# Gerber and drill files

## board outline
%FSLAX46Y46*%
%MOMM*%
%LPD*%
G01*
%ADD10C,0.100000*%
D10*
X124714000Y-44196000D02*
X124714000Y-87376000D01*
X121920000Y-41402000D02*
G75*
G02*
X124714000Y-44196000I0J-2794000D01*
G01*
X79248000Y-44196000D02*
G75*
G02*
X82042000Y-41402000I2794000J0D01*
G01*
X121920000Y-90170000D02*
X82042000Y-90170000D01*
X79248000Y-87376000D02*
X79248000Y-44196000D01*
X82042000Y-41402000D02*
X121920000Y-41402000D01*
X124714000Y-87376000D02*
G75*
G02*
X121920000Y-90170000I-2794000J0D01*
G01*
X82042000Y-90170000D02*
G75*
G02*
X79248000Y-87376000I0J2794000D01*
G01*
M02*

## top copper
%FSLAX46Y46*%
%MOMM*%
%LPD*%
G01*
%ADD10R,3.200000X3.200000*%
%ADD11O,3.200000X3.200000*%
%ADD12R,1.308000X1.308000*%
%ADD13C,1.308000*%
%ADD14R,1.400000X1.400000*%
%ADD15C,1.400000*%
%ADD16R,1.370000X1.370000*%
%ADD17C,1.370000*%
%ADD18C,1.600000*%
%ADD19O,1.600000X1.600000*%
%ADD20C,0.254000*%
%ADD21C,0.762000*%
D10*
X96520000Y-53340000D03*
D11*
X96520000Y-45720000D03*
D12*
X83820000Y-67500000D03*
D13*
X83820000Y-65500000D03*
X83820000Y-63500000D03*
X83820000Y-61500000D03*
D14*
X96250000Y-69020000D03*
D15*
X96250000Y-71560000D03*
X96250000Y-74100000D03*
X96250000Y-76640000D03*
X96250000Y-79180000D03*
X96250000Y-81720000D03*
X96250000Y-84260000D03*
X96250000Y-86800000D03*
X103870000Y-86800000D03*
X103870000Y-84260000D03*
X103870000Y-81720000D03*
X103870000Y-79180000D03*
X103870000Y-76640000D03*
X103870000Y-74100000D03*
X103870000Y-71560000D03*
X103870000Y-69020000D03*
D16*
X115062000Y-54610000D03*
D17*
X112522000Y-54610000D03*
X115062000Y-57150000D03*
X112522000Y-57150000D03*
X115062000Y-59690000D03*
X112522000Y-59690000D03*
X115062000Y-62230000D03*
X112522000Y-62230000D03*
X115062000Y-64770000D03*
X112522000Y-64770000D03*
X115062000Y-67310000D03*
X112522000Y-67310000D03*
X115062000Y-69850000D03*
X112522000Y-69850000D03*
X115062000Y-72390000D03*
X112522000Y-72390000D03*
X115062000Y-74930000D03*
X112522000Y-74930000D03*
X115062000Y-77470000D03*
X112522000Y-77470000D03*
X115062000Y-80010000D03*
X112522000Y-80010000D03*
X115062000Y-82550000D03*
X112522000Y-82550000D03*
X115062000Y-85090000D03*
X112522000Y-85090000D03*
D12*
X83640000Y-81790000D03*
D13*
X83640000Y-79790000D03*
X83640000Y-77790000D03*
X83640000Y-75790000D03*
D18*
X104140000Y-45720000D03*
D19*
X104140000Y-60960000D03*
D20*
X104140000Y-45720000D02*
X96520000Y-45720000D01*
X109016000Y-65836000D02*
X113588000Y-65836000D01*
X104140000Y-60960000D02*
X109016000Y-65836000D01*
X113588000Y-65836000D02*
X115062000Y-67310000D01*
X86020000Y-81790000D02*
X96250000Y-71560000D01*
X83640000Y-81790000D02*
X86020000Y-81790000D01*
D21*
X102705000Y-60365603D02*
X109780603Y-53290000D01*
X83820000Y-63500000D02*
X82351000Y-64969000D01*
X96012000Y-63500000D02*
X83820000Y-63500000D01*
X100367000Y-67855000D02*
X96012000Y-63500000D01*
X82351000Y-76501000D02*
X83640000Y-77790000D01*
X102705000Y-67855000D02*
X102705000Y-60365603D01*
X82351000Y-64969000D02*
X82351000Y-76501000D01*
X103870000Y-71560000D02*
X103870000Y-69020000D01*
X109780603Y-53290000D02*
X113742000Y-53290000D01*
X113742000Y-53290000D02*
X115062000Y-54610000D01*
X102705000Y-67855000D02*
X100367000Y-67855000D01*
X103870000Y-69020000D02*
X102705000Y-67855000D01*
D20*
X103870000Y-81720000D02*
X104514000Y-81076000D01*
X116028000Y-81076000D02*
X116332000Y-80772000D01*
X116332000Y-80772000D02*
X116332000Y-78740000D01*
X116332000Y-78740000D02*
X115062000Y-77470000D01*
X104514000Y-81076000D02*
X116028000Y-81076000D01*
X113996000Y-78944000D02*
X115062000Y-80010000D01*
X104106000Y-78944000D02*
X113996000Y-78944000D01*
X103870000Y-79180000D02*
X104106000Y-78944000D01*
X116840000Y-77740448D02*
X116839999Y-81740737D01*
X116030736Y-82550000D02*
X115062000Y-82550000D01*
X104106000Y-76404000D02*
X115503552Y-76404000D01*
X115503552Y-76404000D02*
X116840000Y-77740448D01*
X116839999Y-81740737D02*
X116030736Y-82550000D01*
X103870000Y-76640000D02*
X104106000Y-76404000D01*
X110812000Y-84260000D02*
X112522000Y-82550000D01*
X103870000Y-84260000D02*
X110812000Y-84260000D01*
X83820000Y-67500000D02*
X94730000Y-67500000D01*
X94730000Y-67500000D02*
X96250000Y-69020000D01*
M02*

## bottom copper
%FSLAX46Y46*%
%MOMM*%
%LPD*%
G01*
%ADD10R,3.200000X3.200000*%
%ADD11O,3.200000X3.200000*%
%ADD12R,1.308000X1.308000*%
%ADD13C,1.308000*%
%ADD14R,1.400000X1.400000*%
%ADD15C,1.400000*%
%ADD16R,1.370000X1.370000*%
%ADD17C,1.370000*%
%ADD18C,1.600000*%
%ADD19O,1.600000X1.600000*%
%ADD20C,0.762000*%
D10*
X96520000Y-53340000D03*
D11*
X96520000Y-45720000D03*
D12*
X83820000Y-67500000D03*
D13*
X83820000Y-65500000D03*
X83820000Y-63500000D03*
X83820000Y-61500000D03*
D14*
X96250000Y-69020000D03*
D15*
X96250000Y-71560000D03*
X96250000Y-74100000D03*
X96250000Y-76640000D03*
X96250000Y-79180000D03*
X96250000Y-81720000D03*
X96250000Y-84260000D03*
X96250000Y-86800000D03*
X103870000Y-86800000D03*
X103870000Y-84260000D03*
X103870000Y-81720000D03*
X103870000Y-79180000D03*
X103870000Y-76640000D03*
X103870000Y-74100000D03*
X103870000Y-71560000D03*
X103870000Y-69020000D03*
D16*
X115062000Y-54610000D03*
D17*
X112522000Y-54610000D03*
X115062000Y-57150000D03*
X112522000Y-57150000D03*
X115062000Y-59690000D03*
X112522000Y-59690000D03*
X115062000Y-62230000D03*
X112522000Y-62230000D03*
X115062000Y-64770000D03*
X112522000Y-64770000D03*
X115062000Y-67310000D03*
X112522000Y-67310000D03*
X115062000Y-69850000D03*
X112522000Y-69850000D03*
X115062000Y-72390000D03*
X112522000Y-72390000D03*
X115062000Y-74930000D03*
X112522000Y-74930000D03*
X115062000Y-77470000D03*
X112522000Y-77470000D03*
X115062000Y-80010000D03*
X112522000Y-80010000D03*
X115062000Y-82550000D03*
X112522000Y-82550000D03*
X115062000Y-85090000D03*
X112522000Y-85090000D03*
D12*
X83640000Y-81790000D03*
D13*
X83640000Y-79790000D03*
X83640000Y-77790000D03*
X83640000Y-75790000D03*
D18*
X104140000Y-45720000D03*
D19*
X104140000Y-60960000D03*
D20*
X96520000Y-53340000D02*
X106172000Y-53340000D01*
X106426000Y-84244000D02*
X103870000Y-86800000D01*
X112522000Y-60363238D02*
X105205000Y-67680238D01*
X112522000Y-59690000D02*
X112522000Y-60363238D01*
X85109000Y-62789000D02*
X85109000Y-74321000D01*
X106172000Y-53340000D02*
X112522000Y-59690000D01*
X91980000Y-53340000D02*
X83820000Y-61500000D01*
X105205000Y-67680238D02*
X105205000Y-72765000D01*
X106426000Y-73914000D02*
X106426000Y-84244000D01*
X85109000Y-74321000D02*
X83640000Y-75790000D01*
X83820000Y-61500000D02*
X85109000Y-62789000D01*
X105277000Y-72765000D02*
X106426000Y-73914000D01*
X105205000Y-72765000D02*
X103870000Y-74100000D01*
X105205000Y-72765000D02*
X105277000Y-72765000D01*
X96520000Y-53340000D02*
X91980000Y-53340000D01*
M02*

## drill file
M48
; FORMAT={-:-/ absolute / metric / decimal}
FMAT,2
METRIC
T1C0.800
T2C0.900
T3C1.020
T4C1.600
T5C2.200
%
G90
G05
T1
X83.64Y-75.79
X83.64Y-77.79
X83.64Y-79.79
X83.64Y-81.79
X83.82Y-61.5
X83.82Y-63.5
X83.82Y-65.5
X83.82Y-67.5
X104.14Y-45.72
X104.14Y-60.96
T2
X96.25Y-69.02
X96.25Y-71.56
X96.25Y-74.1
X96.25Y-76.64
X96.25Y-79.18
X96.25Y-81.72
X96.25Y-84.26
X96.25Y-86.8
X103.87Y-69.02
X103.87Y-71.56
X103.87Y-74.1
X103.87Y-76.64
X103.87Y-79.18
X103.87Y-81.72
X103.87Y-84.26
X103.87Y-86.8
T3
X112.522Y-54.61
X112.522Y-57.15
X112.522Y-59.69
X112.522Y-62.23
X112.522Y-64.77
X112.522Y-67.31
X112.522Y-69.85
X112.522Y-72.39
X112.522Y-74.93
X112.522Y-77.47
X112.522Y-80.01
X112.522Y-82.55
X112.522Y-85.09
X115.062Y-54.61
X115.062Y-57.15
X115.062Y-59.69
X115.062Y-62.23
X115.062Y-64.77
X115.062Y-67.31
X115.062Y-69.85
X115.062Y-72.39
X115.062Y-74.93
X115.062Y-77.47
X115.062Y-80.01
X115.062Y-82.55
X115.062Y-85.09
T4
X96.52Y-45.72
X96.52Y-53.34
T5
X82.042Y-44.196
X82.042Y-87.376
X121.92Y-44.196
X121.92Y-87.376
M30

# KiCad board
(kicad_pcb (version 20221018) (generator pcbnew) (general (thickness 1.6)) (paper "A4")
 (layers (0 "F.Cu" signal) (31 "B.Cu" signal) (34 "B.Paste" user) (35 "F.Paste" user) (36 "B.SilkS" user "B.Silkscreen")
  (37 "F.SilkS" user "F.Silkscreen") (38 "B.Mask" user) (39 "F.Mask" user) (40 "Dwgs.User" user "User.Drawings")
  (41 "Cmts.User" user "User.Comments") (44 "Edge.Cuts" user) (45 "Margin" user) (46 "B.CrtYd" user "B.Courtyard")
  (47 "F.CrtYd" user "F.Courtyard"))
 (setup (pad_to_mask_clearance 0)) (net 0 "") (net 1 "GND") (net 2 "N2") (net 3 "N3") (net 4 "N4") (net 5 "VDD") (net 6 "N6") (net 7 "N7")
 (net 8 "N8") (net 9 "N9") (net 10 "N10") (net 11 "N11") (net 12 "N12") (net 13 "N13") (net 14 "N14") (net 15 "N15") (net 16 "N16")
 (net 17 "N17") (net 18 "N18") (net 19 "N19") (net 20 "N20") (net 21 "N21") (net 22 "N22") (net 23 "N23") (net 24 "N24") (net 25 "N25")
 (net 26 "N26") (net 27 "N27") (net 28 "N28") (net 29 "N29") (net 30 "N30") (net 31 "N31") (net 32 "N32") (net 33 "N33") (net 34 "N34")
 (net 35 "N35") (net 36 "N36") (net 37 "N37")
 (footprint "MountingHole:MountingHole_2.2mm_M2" (layer "F.Cu") (at 121.92 44.196)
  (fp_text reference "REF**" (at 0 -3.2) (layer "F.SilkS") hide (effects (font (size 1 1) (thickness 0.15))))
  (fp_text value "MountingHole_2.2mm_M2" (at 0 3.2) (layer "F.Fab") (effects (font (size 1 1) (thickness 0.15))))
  (pad "" np_thru_hole circle (at 0 0) (size 2.2 2.2) (drill 2.2) (layers "*.Cu" "*.Mask")))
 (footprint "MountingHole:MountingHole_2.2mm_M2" (layer "F.Cu") (at 82.042 87.376)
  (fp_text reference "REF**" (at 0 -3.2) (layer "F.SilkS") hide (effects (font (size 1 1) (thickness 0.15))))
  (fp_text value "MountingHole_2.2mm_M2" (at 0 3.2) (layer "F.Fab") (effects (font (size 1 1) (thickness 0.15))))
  (pad "" np_thru_hole circle (at 0 0) (size 2.2 2.2) (drill 2.2) (layers "*.Cu" "*.Mask")))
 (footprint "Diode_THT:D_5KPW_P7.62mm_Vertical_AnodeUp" (layer "F.Cu") (at 96.52 53.34 90)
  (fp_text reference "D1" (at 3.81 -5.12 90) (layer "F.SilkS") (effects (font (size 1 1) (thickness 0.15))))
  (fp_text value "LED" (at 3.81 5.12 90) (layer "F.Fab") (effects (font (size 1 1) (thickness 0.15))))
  (pad "1" thru_hole rect (at 0 0 90) (size 3.2 3.2) (drill 1.6) (layers "*.Cu" "*.Mask") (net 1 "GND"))
  (pad "2" thru_hole oval (at 7.62 0 90) (size 3.2 3.2) (drill 1.6) (layers "*.Cu" "*.Mask") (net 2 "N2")))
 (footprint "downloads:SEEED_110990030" (layer "F.Cu") (at 83.82 64.5 90)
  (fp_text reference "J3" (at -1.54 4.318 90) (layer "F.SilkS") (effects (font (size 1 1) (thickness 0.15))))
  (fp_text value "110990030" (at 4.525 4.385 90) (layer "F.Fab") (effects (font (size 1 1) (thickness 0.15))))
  (pad "1" thru_hole rect (at -3 0 90) (size 1.308 1.308) (drill 0.8) (layers "*.Cu" "*.Mask") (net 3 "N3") (solder_mask_margin 0.102))
  (pad "2" thru_hole circle (at -1 0 90) (size 1.308 1.308) (drill 0.8) (layers "*.Cu" "*.Mask") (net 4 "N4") (solder_mask_margin 0.102))
  (pad "3" thru_hole circle (at 1 0 90) (size 1.308 1.308) (drill 0.8) (layers "*.Cu" "*.Mask") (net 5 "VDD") (solder_mask_margin 0.102))
  (pad "4" thru_hole circle (at 3 0 90) (size 1.308 1.308) (drill 0.8) (layers "*.Cu" "*.Mask") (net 1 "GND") (solder_mask_margin 0.102)))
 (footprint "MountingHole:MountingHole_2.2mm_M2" (layer "F.Cu") (at 82.042 44.196)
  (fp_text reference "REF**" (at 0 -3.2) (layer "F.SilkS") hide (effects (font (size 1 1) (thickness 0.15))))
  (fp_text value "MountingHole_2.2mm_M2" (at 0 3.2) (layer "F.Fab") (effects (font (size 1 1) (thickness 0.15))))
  (pad "" np_thru_hole circle (at 0 0) (size 2.2 2.2) (drill 2.2) (layers "*.Cu" "*.Mask")))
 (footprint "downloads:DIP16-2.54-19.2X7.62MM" (layer "F.Cu") (at 100.06 77.91 -90)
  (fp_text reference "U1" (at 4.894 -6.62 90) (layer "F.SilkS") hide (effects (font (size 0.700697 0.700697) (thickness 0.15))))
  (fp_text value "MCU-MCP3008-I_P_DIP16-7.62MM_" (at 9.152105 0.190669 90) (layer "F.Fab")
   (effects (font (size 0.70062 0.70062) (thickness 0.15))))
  (pad "1" thru_hole rect (at -8.89 3.81 270) (size 1.4 1.4) (drill 0.9) (layers "*.Cu" "*.Mask") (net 3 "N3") (solder_mask_margin 0.102))
  (pad "2" thru_hole circle (at -6.35 3.81 270) (size 1.4 1.4) (drill 0.9) (layers "*.Cu" "*.Mask") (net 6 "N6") (solder_mask_margin 0.102))
  (pad "3" thru_hole circle (at -3.81 3.81 270) (size 1.4 1.4) (drill 0.9) (layers "*.Cu" "*.Mask") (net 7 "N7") (solder_mask_margin 0.102))
  (pad "4" thru_hole circle (at -1.27 3.81 270) (size 1.4 1.4) (drill 0.9) (layers "*.Cu" "*.Mask") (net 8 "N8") (solder_mask_margin 0.102))
  (pad "5" thru_hole circle (at 1.27 3.81 270) (size 1.4 1.4) (drill 0.9) (layers "*.Cu" "*.Mask") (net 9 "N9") (solder_mask_margin 0.102))
  (pad "6" thru_hole circle (at 3.81 3.81 270) (size 1.4 1.4) (drill 0.9) (layers "*.Cu" "*.Mask") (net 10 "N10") (solder_mask_margin 0.102))
  (pad "7" thru_hole circle (at 6.35 3.81 270) (size 1.4 1.4) (drill 0.9) (layers "*.Cu" "*.Mask") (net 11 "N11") (solder_mask_margin 0.102))
  (pad "8" thru_hole circle (at 8.89 3.81 270) (size 1.4 1.4) (drill 0.9) (layers "*.Cu" "*.Mask") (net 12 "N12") (solder_mask_margin 0.102))
  (pad "9" thru_hole circle (at 8.89 -3.81 270) (size 1.4 1.4) (drill 0.9) (layers "*.Cu" "*.Mask") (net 1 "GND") (solder_mask_margin 0.102))
  (pad "10" thru_hole circle (at 6.35 -3.81 270) (size 1.4 1.4) (drill 0.9) (layers "*.Cu" "*.Mask") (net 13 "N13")
   (solder_mask_margin 0.102))
  (pad "11" thru_hole circle (at 3.81 -3.81 270) (size 1.4 1.4) (drill 0.9) (layers "*.Cu" "*.Mask") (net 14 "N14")
   (solder_mask_margin 0.102))
  (pad "12" thru_hole circle (at 1.27 -3.81 270) (size 1.4 1.4) (drill 0.9) (layers "*.Cu" "*.Mask") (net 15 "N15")
   (solder_mask_margin 0.102))
  (pad "13" thru_hole circle (at -1.27 -3.81 270) (size 1.4 1.4) (drill 0.9) (layers "*.Cu" "*.Mask") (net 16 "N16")
   (solder_mask_margin 0.102))
  (pad "14" thru_hole circle (at -3.81 -3.81 270) (size 1.4 1.4) (drill 0.9) (layers "*.Cu" "*.Mask") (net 1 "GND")
   (solder_mask_margin 0.102))
  (pad "15" thru_hole circle (at -6.35 -3.81 270) (size 1.4 1.4) (drill 0.9) (layers "*.Cu" "*.Mask") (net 5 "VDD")
   (solder_mask_margin 0.102))
  (pad "16" thru_hole circle (at -8.89 -3.81 270) (size 1.4 1.4) (drill 0.9) (layers "*.Cu" "*.Mask") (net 5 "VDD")
   (solder_mask_margin 0.102)))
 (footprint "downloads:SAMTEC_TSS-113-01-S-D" (layer "F.Cu") (at 112.912 54.61 -90)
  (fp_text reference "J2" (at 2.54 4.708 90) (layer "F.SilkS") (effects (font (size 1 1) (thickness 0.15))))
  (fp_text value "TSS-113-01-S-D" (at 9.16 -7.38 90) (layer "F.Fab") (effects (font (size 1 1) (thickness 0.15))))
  (pad "01" thru_hole rect (at 0 -2.15 270) (size 1.37 1.37) (drill 1.02) (layers "*.Cu" "*.Mask") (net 5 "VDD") (solder_mask_margin 0.102))
  (pad "02" thru_hole circle (at 0 0.39 270) (size 1.37 1.37) (drill 1.02) (layers "*.Cu" "*.Mask") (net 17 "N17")
   (solder_mask_margin 0.102))
  (pad "03" thru_hole circle (at 2.54 -2.15 270) (size 1.37 1.37) (drill 1.02) (layers "*.Cu" "*.Mask") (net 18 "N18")
   (solder_mask_margin 0.102))
  (pad "04" thru_hole circle (at 2.54 0.39 270) (size 1.37 1.37) (drill 1.02) (layers "*.Cu" "*.Mask") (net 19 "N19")
   (solder_mask_margin 0.102))
  (pad "05" thru_hole circle (at 5.08 -2.15 270) (size 1.37 1.37) (drill 1.02) (layers "*.Cu" "*.Mask") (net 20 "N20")
   (solder_mask_margin 0.102))
  (pad "06" thru_hole circle (at 5.08 0.39 270) (size 1.37 1.37) (drill 1.02) (layers "*.Cu" "*.Mask") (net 1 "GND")
   (solder_mask_margin 0.102))
  (pad "07" thru_hole circle (at 7.62 -2.15 270) (size 1.37 1.37) (drill 1.02) (layers "*.Cu" "*.Mask") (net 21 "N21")
   (solder_mask_margin 0.102))
  (pad "08" thru_hole circle (at 7.62 0.39 270) (size 1.37 1.37) (drill 1.02) (layers "*.Cu" "*.Mask") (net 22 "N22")
   (solder_mask_margin 0.102))
  (pad "09" thru_hole circle (at 10.16 -2.15 270) (size 1.37 1.37) (drill 1.02) (layers "*.Cu" "*.Mask") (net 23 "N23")
   (solder_mask_margin 0.102))
  (pad "10" thru_hole circle (at 10.16 0.39 270) (size 1.37 1.37) (drill 1.02) (layers "*.Cu" "*.Mask") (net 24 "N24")
   (solder_mask_margin 0.102))
  (pad "11" thru_hole circle (at 12.7 -2.15 270) (size 1.37 1.37) (drill 1.02) (layers "*.Cu" "*.Mask") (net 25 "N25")
   (solder_mask_margin 0.102))
  (pad "12" thru_hole circle (at 12.7 0.39 270) (size 1.37 1.37) (drill 1.02) (layers "*.Cu" "*.Mask") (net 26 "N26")
   (solder_mask_margin 0.102))
  (pad "13" thru_hole circle (at 15.24 -2.15 270) (size 1.37 1.37) (drill 1.02) (layers "*.Cu" "*.Mask") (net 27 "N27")
   (solder_mask_margin 0.102))
  (pad "14" thru_hole circle (at 15.24 0.39 270) (size 1.37 1.37) (drill 1.02) (layers "*.Cu" "*.Mask") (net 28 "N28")
   (solder_mask_margin 0.102))
  (pad "15" thru_hole circle (at 17.78 -2.15 270) (size 1.37 1.37) (drill 1.02) (layers "*.Cu" "*.Mask") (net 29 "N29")
   (solder_mask_margin 0.102))
  (pad "16" thru_hole circle (at 17.78 0.39 270) (size 1.37 1.37) (drill 1.02) (layers "*.Cu" "*.Mask") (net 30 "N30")
   (solder_mask_margin 0.102))
  (pad "17" thru_hole circle (at 20.32 -2.15 270) (size 1.37 1.37) (drill 1.02) (layers "*.Cu" "*.Mask") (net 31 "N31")
   (solder_mask_margin 0.102))
  (pad "18" thru_hole circle (at 20.32 0.39 270) (size 1.37 1.37) (drill 1.02) (layers "*.Cu" "*.Mask") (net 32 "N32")
   (solder_mask_margin 0.102))
  (pad "19" thru_hole circle (at 22.86 -2.15 270) (size 1.37 1.37) (drill 1.02) (layers "*.Cu" "*.Mask") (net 14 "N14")
   (solder_mask_margin 0.102))
  (pad "20" thru_hole circle (at 22.86 0.39 270) (size 1.37 1.37) (drill 1.02) (layers "*.Cu" "*.Mask") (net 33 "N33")
   (solder_mask_margin 0.102))
  (pad "21" thru_hole circle (at 25.4 -2.15 270) (size 1.37 1.37) (drill 1.02) (layers "*.Cu" "*.Mask") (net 15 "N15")
   (solder_mask_margin 0.102))
  (pad "22" thru_hole circle (at 25.4 0.39 270) (size 1.37 1.37) (drill 1.02) (layers "*.Cu" "*.Mask") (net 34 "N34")
   (solder_mask_margin 0.102))
  (pad "23" thru_hole circle (at 27.94 -2.15 270) (size 1.37 1.37) (drill 1.02) (layers "*.Cu" "*.Mask") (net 16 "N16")
   (solder_mask_margin 0.102))
  (pad "24" thru_hole circle (at 27.94 0.39 270) (size 1.37 1.37) (drill 1.02) (layers "*.Cu" "*.Mask") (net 13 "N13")
   (solder_mask_margin 0.102))
  (pad "25" thru_hole circle (at 30.48 -2.15 270) (size 1.37 1.37) (drill 1.02) (layers "*.Cu" "*.Mask") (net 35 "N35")
   (solder_mask_margin 0.102))
  (pad "26" thru_hole circle (at 30.48 0.39 270) (size 1.37 1.37) (drill 1.02) (layers "*.Cu" "*.Mask") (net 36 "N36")
   (solder_mask_margin 0.102)))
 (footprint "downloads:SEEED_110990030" (layer "F.Cu") (at 83.64 78.79 90)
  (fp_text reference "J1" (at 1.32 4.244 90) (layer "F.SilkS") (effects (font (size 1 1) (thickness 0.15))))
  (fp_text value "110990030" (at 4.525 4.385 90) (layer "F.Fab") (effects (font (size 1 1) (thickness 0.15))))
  (pad "1" thru_hole rect (at -3 0 90) (size 1.308 1.308) (drill 0.8) (layers "*.Cu" "*.Mask") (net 6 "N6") (solder_mask_margin 0.102))
  (pad "2" thru_hole circle (at -1 0 90) (size 1.308 1.308) (drill 0.8) (layers "*.Cu" "*.Mask") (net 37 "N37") (solder_mask_margin 0.102))
  (pad "3" thru_hole circle (at 1 0 90) (size 1.308 1.308) (drill 0.8) (layers "*.Cu" "*.Mask") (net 5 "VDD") (solder_mask_margin 0.102))
  (pad "4" thru_hole circle (at 3 0 90) (size 1.308 1.308) (drill 0.8) (layers "*.Cu" "*.Mask") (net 1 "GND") (solder_mask_margin 0.102)))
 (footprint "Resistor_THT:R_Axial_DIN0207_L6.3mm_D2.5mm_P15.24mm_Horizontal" (layer "F.Cu") (at 104.14 45.72 -90)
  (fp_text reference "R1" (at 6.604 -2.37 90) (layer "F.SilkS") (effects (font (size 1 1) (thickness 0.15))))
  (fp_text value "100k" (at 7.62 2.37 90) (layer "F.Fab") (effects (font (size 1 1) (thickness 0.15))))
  (pad "1" thru_hole circle (at 0 0 270) (size 1.6 1.6) (drill 0.8) (layers "*.Cu" "*.Mask") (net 2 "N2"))
  (pad "2" thru_hole oval (at 15.24 0 270) (size 1.6 1.6) (drill 0.8) (layers "*.Cu" "*.Mask") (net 25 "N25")))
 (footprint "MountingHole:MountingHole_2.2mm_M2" (layer "F.Cu") (at 121.92 87.376)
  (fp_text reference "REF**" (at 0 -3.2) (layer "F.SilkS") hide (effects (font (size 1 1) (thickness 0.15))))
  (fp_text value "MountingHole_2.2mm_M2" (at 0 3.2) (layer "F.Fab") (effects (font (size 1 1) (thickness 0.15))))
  (pad "" np_thru_hole circle (at 0 0) (size 2.2 2.2) (drill 2.2) (layers "*.Cu" "*.Mask")))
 (gr_line (start 124.714 44.196) (end 124.714 87.376) (stroke (width 0.1) (type default)) (layer "Edge.Cuts"))
 (gr_arc (start 121.92 41.402) (mid 123.895656 42.220344) (end 124.714 44.196) (stroke (width 0.1) (type default)) (layer "Edge.Cuts"))
 (gr_arc (start 79.248 44.196) (mid 80.066344 42.220344) (end 82.042 41.402) (stroke (width 0.1) (type default)) (layer "Edge.Cuts"))
 (gr_line (start 121.92 90.17) (end 82.042 90.17) (stroke (width 0.1) (type default)) (layer "Edge.Cuts"))
 (gr_line (start 79.248 87.376) (end 79.248 44.196) (stroke (width 0.1) (type default)) (layer "Edge.Cuts"))
 (gr_line (start 82.042 41.402) (end 121.92 41.402) (stroke (width 0.1) (type default)) (layer "Edge.Cuts"))
 (gr_arc (start 124.714 87.376) (mid 123.895656 89.351656) (end 121.92 90.17) (stroke (width 0.1) (type default)) (layer "Edge.Cuts"))
 (gr_arc (start 82.042 90.17) (mid 80.066344 89.351656) (end 79.248 87.376) (stroke (width 0.1) (type default)) (layer "Edge.Cuts"))
 (segment (start 96.52 53.34) (end 106.172 53.34) (width 0.762) (layer "B.Cu") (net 1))
 (segment (start 106.426 84.244) (end 103.87 86.8) (width 0.762) (layer "B.Cu") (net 1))
 (segment (start 112.522 60.363238) (end 105.205 67.680238) (width 0.762) (layer "B.Cu") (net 1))
 (segment (start 112.522 59.69) (end 112.522 60.363238) (width 0.762) (layer "B.Cu") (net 1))
 (segment (start 85.109 62.789) (end 85.109 74.321) (width 0.762) (layer "B.Cu") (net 1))
 (segment (start 106.172 53.34) (end 112.522 59.69) (width 0.762) (layer "B.Cu") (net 1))
 (segment (start 91.98 53.34) (end 83.82 61.5) (width 0.762) (layer "B.Cu") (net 1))
 (segment (start 105.205 67.680238) (end 105.205 72.765) (width 0.762) (layer "B.Cu") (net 1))
 (segment (start 106.426 73.914) (end 106.426 84.244) (width 0.762) (layer "B.Cu") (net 1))
 (segment (start 85.109 74.321) (end 83.64 75.79) (width 0.762) (layer "B.Cu") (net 1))
 (segment (start 83.82 61.5) (end 85.109 62.789) (width 0.762) (layer "B.Cu") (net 1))
 (segment (start 105.277 72.765) (end 106.426 73.914) (width 0.762) (layer "B.Cu") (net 1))
 (segment (start 105.205 72.765) (end 103.87 74.1) (width 0.762) (layer "B.Cu") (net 1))
 (segment (start 105.205 72.765) (end 105.277 72.765) (width 0.762) (layer "B.Cu") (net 1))
 (segment (start 96.52 53.34) (end 91.98 53.34) (width 0.762) (layer "B.Cu") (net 1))
 (segment (start 104.14 45.72) (end 96.52 45.72) (width 0.254) (layer "F.Cu") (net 2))
 (segment (start 109.016 65.836) (end 113.588 65.836) (width 0.254) (layer "F.Cu") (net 25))
 (segment (start 104.14 60.96) (end 109.016 65.836) (width 0.254) (layer "F.Cu") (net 25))
 (segment (start 113.588 65.836) (end 115.062 67.31) (width 0.254) (layer "F.Cu") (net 25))
 (segment (start 86.02 81.79) (end 96.25 71.56) (width 0.254) (layer "F.Cu") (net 6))
 (segment (start 83.64 81.79) (end 86.02 81.79) (width 0.254) (layer "F.Cu") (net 6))
 (segment (start 102.705 60.365603) (end 109.780603 53.29) (width 0.762) (layer "F.Cu") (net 5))
 (segment (start 83.82 63.5) (end 82.351 64.969) (width 0.762) (layer "F.Cu") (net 5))
 (segment (start 96.012 63.5) (end 83.82 63.5) (width 0.762) (layer "F.Cu") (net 5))
 (segment (start 100.367 67.855) (end 96.012 63.5) (width 0.762) (layer "F.Cu") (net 5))
 (segment (start 82.351 76.501) (end 83.64 77.79) (width 0.762) (layer "F.Cu") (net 5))
 (segment (start 102.705 67.855) (end 102.705 60.365603) (width 0.762) (layer "F.Cu") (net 5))
 (segment (start 82.351 64.969) (end 82.351 76.501) (width 0.762) (layer "F.Cu") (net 5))
 (segment (start 103.87 71.56) (end 103.87 69.02) (width 0.762) (layer "F.Cu") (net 5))
 (segment (start 109.780603 53.29) (end 113.742 53.29) (width 0.762) (layer "F.Cu") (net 5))
 (segment (start 113.742 53.29) (end 115.062 54.61) (width 0.762) (layer "F.Cu") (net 5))
 (segment (start 102.705 67.855) (end 100.367 67.855) (width 0.762) (layer "F.Cu") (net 5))
 (segment (start 103.87 69.02) (end 102.705 67.855) (width 0.762) (layer "F.Cu") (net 5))
 (segment (start 103.87 81.72) (end 104.514 81.076) (width 0.254) (layer "F.Cu") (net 14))
 (segment (start 116.028 81.076) (end 116.332 80.772) (width 0.254) (layer "F.Cu") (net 14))
 (segment (start 116.332 80.772) (end 116.332 78.74) (width 0.254) (layer "F.Cu") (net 14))
 (segment (start 116.332 78.74) (end 115.062 77.47) (width 0.254) (layer "F.Cu") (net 14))
 (segment (start 104.514 81.076) (end 116.028 81.076) (width 0.254) (layer "F.Cu") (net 14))
 (segment (start 113.996 78.944) (end 115.062 80.01) (width 0.254) (layer "F.Cu") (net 15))
 (segment (start 104.106 78.944) (end 113.996 78.944) (width 0.254) (layer "F.Cu") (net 15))
 (segment (start 103.87 79.18) (end 104.106 78.944) (width 0.254) (layer "F.Cu") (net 15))
 (segment (start 116.84 77.740448) (end 116.839999 81.740737) (width 0.254) (layer "F.Cu") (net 16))
 (segment (start 116.030736 82.55) (end 115.062 82.55) (width 0.254) (layer "F.Cu") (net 16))
 (segment (start 104.106 76.404) (end 115.503552 76.404) (width 0.254) (layer "F.Cu") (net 16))
 (segment (start 115.503552 76.404) (end 116.84 77.740448) (width 0.254) (layer "F.Cu") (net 16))
 (segment (start 116.839999 81.740737) (end 116.030736 82.55) (width 0.254) (layer "F.Cu") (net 16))
 (segment (start 103.87 76.64) (end 104.106 76.404) (width 0.254) (layer "F.Cu") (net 16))
 (segment (start 110.812 84.26) (end 112.522 82.55) (width 0.254) (layer "F.Cu") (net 13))
 (segment (start 103.87 84.26) (end 110.812 84.26) (width 0.254) (layer "F.Cu") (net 13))
 (segment (start 83.82 67.5) (end 94.73 67.5) (width 0.254) (layer "F.Cu") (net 3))
 (segment (start 94.73 67.5) (end 96.25 69.02) (width 0.254) (layer "F.Cu") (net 3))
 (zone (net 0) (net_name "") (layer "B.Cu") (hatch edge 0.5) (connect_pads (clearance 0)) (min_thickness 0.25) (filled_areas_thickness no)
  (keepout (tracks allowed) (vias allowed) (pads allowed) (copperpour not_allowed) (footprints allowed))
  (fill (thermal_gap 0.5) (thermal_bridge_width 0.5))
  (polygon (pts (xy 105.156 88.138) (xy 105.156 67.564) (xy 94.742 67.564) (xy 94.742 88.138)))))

